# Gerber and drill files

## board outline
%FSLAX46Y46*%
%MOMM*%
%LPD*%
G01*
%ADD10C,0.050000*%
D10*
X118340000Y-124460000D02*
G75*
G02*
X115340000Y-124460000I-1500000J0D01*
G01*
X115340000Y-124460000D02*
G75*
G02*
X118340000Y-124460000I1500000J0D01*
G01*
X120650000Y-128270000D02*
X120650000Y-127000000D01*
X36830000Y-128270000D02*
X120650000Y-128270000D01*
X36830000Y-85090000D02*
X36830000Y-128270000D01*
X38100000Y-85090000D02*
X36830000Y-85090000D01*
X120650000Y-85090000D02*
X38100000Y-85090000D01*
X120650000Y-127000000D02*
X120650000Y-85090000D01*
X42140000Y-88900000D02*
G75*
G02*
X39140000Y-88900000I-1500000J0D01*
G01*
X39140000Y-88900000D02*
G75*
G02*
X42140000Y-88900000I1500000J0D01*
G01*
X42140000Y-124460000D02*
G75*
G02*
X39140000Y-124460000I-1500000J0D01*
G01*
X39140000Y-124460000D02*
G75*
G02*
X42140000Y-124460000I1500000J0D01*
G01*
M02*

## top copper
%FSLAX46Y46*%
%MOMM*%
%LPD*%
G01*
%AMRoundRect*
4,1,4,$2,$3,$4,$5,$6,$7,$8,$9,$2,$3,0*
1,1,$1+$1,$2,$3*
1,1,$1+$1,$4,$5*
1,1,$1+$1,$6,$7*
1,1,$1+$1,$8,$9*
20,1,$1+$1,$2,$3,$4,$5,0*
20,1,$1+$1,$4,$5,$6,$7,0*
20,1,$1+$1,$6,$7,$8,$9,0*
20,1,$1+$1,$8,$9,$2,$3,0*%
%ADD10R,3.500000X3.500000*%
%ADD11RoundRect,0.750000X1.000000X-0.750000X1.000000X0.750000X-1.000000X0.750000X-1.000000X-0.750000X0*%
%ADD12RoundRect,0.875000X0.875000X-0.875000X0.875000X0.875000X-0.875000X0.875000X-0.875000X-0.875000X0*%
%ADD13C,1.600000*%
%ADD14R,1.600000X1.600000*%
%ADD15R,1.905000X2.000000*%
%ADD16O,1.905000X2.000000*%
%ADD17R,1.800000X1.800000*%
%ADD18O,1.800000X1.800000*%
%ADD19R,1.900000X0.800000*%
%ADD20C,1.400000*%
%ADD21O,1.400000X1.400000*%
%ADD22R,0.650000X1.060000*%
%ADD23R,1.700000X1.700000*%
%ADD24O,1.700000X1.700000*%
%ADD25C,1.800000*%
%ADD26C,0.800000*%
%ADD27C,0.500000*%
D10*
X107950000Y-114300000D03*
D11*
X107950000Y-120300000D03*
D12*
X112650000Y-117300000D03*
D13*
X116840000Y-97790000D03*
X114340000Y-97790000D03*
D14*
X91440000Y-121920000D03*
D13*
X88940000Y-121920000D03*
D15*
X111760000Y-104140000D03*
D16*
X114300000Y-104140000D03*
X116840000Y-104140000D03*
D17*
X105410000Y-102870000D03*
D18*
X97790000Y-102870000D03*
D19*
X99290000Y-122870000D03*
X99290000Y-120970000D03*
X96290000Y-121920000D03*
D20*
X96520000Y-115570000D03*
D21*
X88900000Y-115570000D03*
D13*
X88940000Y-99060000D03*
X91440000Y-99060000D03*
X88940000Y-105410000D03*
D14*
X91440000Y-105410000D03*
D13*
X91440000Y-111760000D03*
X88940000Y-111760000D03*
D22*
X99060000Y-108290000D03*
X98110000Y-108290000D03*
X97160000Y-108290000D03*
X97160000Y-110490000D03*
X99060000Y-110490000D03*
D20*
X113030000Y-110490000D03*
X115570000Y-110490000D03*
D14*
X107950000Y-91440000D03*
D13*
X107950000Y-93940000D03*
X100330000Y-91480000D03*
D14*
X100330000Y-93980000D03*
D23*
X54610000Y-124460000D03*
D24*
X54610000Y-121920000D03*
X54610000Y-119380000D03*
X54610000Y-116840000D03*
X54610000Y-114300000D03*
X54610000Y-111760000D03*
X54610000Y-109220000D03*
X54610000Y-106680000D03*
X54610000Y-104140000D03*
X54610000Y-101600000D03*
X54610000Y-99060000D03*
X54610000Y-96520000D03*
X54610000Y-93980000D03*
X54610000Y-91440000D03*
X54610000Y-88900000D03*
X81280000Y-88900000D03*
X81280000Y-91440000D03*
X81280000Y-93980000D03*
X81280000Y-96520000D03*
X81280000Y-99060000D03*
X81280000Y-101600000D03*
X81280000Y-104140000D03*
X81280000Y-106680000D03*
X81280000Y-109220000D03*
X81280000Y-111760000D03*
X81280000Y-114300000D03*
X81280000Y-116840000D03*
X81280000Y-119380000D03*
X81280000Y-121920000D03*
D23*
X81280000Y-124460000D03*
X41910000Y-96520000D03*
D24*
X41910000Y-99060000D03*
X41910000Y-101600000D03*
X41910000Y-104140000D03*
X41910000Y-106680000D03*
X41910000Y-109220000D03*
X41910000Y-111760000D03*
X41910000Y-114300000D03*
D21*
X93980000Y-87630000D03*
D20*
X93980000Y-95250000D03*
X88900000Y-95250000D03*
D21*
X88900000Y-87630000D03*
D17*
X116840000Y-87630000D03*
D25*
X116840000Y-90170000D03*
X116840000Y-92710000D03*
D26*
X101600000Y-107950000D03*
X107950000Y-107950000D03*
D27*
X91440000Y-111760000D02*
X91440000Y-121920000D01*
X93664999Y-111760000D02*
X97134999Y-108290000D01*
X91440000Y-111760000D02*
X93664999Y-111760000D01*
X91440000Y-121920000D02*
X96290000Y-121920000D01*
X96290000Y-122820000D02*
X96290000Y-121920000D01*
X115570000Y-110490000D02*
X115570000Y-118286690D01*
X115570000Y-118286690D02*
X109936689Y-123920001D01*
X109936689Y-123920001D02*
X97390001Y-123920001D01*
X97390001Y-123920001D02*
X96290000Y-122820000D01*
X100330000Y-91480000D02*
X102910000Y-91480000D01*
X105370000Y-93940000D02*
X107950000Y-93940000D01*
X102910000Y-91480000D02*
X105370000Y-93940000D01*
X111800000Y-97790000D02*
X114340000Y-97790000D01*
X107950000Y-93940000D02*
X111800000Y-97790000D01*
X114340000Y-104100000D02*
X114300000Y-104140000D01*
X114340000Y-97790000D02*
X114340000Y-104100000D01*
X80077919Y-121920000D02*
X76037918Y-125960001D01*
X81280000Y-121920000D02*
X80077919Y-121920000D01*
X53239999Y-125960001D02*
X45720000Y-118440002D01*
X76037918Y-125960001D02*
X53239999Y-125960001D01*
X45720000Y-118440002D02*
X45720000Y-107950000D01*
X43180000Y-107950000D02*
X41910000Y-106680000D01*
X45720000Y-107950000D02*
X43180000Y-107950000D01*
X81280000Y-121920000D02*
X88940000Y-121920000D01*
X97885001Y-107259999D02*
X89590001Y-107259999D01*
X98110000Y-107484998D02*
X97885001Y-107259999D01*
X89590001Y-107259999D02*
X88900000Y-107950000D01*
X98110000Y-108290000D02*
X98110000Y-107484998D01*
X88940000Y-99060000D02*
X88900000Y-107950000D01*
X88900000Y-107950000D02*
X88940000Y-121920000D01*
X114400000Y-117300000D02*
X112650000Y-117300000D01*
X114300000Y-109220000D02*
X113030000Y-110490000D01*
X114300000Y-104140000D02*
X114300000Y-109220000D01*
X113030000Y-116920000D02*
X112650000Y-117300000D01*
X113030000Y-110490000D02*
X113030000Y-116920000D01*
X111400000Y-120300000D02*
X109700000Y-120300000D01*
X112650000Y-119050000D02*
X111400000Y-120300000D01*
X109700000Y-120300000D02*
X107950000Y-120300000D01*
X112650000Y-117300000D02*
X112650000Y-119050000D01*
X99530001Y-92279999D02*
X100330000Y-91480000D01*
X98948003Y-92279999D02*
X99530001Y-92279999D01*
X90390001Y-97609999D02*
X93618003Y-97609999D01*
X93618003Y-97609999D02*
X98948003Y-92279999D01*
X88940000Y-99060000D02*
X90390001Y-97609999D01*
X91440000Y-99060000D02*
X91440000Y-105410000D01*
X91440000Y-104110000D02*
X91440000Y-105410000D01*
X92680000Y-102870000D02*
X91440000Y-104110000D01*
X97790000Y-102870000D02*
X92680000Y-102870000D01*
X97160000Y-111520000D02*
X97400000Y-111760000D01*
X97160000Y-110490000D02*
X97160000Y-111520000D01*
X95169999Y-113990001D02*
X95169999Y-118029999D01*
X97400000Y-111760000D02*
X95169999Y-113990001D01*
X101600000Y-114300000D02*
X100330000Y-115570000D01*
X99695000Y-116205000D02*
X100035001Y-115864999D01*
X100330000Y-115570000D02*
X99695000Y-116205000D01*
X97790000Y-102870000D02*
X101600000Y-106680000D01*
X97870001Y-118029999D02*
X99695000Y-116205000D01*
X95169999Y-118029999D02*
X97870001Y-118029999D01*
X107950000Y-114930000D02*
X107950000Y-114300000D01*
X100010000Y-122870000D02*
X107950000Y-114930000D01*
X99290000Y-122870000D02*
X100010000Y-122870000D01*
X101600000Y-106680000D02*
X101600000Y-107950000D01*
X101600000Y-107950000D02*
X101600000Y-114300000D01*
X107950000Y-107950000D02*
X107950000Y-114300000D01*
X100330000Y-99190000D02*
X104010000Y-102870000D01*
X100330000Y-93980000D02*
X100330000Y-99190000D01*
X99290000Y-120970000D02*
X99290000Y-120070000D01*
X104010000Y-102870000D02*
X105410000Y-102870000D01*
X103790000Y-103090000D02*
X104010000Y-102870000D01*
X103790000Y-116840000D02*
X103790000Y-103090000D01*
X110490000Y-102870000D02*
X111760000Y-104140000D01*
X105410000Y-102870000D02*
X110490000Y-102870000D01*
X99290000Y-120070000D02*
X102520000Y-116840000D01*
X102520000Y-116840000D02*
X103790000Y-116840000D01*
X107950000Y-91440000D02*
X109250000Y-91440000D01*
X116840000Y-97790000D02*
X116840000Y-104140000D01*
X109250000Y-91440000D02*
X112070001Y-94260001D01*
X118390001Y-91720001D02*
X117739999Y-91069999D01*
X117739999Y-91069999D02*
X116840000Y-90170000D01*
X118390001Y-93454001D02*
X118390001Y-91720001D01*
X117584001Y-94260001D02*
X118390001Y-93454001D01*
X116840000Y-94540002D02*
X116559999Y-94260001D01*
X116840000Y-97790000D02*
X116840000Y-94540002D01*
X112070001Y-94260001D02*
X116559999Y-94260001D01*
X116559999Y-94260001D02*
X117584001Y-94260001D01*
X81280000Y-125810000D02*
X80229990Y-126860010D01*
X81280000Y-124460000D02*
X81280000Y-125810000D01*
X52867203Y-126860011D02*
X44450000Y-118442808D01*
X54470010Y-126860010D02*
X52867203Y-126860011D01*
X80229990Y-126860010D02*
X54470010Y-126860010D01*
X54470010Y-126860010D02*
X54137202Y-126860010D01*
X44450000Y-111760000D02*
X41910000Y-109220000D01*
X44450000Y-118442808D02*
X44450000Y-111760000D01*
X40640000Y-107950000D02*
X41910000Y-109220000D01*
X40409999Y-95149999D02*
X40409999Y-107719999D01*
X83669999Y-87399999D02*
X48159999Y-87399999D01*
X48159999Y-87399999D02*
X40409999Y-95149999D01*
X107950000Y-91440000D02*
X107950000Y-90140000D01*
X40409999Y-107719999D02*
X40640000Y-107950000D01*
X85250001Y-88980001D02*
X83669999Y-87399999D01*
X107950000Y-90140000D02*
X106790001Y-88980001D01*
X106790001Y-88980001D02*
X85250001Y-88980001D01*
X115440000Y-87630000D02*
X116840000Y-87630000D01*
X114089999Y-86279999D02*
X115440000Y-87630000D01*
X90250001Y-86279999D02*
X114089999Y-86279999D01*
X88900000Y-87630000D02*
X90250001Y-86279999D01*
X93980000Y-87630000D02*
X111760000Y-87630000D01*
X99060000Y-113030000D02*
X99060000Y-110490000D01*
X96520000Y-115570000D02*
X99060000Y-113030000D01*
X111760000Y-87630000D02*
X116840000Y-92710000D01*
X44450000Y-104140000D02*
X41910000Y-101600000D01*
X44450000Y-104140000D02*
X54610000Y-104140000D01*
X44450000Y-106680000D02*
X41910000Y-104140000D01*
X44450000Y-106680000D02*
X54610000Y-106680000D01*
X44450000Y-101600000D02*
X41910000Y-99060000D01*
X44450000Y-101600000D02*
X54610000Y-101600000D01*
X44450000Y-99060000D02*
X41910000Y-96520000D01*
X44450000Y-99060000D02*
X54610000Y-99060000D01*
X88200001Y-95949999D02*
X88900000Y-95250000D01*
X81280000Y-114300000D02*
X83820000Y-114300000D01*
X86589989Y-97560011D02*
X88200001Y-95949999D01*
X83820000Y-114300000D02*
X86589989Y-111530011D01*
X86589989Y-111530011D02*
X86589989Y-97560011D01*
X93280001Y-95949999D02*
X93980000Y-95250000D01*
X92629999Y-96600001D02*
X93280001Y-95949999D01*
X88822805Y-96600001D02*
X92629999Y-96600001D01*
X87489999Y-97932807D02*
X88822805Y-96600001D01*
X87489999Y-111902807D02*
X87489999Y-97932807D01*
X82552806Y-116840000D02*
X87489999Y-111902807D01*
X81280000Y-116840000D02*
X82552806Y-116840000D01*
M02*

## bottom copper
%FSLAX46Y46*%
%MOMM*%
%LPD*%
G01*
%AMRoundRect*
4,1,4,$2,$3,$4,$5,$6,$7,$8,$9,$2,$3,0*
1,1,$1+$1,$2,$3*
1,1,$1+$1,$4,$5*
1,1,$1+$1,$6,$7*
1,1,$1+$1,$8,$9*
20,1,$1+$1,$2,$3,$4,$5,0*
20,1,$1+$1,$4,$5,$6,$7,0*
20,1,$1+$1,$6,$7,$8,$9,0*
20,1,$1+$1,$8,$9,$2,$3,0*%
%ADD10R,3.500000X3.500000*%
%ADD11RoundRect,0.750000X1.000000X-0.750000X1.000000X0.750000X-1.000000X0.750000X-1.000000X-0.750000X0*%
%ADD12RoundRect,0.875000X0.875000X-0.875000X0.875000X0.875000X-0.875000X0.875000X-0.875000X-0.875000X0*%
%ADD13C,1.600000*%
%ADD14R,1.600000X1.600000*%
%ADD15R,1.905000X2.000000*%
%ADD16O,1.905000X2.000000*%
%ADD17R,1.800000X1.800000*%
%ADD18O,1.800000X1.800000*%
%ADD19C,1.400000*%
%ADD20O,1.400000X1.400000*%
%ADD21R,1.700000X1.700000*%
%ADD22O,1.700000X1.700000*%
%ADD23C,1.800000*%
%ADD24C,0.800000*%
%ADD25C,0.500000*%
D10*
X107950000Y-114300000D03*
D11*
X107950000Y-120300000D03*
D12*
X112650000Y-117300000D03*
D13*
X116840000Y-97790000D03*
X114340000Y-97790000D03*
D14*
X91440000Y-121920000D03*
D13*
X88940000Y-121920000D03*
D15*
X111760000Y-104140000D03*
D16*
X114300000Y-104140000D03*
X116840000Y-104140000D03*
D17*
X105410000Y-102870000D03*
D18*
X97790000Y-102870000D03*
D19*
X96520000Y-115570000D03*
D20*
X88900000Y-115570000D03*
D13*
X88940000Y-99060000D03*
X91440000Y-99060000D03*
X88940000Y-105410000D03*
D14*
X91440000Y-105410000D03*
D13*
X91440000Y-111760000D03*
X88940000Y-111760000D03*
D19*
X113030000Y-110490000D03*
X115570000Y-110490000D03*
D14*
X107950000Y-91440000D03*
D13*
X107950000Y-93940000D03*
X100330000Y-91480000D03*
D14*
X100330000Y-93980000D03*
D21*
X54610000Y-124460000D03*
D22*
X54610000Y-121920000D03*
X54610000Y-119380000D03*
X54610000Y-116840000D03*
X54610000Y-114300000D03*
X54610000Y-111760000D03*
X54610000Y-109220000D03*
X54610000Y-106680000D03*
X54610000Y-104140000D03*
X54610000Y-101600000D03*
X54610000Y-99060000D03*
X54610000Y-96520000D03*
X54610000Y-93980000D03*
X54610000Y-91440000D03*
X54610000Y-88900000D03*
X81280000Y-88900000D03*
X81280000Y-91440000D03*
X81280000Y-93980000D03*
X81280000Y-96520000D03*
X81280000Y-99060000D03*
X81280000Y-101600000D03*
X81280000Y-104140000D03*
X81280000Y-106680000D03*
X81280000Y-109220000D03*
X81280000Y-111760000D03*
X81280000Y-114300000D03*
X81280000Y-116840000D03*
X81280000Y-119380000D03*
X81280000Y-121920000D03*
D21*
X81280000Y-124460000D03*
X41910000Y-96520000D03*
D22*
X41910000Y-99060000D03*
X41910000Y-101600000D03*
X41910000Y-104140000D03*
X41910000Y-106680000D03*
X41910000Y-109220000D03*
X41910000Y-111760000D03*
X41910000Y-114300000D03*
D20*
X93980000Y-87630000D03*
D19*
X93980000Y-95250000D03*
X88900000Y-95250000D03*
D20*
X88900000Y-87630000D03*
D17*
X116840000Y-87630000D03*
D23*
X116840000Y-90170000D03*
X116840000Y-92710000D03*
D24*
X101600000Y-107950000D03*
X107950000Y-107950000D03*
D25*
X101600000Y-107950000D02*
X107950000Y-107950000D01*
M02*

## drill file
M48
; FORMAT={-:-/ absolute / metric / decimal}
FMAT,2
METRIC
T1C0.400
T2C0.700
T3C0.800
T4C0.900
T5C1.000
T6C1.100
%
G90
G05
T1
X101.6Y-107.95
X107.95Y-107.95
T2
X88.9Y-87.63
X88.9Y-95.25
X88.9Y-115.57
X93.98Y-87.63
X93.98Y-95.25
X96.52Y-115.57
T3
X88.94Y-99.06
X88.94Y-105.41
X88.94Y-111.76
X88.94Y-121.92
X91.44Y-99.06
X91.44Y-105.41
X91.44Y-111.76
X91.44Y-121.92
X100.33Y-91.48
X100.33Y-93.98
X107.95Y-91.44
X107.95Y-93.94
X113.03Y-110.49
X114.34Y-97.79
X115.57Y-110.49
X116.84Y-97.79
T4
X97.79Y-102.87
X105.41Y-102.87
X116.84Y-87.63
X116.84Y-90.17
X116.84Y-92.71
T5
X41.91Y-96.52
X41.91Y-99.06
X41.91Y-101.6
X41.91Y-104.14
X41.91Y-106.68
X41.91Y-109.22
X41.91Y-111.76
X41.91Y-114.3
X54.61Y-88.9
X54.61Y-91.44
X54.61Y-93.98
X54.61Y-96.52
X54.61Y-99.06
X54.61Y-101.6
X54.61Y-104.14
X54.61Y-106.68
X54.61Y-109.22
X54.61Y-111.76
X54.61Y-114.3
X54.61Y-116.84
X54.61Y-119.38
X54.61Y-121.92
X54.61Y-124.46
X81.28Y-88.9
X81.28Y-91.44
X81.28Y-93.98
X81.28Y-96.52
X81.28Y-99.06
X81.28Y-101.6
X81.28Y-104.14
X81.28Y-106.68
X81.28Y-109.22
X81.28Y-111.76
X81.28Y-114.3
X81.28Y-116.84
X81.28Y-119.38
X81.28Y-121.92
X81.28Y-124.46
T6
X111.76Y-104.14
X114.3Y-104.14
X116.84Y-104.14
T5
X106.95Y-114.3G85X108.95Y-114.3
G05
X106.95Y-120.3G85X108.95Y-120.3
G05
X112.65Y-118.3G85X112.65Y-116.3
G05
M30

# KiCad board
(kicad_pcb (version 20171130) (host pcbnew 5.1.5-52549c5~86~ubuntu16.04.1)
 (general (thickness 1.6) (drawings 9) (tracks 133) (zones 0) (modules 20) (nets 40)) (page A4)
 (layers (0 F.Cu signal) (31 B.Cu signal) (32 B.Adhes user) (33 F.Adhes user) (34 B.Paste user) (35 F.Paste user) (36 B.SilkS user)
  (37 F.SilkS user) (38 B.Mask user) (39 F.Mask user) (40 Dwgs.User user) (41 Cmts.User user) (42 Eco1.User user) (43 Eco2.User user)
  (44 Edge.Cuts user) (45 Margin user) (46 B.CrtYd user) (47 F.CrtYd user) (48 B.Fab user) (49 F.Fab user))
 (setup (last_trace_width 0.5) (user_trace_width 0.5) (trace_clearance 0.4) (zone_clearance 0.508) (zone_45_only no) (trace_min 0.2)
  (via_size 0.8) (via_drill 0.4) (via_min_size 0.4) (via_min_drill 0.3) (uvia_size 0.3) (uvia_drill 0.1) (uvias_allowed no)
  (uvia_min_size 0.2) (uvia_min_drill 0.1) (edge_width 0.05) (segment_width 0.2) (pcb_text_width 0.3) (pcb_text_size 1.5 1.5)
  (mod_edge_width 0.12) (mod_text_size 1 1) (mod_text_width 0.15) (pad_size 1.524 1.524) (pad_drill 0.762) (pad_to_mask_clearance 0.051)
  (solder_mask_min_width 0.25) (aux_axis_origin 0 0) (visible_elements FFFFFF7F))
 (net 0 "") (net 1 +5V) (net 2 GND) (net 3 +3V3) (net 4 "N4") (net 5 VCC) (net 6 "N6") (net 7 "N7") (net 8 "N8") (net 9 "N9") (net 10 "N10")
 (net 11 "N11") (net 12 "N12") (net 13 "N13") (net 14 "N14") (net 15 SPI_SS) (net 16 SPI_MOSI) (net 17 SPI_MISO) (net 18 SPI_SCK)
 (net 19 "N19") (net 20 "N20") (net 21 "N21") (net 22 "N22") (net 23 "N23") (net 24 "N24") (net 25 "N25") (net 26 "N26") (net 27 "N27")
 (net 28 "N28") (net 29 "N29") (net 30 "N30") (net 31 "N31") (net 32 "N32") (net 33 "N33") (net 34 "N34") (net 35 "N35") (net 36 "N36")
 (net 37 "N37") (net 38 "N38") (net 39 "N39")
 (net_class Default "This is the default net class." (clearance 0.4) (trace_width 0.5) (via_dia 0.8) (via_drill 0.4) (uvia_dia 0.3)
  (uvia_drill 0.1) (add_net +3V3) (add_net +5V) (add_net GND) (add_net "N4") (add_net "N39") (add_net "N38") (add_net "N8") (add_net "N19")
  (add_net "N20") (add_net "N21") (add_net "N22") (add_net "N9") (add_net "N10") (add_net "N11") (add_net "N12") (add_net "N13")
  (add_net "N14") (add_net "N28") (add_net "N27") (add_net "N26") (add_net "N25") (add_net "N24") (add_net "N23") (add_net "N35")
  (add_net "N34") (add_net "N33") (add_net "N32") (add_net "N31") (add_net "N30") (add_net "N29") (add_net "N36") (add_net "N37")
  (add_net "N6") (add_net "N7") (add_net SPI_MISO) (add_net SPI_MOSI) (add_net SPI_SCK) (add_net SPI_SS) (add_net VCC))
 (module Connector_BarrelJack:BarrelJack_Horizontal (layer F.Cu) (at 107.95 114.3 90)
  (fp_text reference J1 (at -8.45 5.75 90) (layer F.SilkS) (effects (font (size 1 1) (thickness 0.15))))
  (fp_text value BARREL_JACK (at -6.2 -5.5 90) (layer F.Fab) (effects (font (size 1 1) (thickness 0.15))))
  (pad 1 thru_hole rect (at 0 0 90) (size 3.5 3.5) (drill oval 1 3) (layers *.Cu *.Mask) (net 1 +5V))
  (pad 2 thru_hole roundrect (at -6 0 90) (size 3 3.5) (drill oval 1 3) (layers *.Cu *.Mask) (roundrect_rratio 0.25) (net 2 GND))
  (pad 3 thru_hole roundrect (at -3 4.7 90) (size 3.5 3.5) (drill oval 3 1) (layers *.Cu *.Mask) (roundrect_rratio 0.25) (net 2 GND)))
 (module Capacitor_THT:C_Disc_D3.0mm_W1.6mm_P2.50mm (layer F.Cu) (at 116.84 97.79 180)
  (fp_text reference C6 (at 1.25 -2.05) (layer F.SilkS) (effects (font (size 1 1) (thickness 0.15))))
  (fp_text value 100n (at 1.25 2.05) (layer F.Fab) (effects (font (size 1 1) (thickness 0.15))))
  (pad 1 thru_hole circle (at 0 0 180) (size 1.6 1.6) (drill 0.8) (layers *.Cu *.Mask) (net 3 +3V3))
  (pad 2 thru_hole circle (at 2.5 0 180) (size 1.6 1.6) (drill 0.8) (layers *.Cu *.Mask) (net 2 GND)))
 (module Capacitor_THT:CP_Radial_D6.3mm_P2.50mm (layer F.Cu) (at 91.44 121.92 180)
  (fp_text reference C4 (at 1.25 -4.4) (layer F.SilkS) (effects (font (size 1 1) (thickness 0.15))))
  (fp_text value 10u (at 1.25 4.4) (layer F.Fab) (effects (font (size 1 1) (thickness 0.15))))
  (pad 1 thru_hole rect (at 0 0 180) (size 1.6 1.6) (drill 0.8) (layers *.Cu *.Mask) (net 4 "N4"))
  (pad 2 thru_hole circle (at 2.5 0 180) (size 1.6 1.6) (drill 0.8) (layers *.Cu *.Mask) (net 2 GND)))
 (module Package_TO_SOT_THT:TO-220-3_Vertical (layer F.Cu) (at 111.76 104.14)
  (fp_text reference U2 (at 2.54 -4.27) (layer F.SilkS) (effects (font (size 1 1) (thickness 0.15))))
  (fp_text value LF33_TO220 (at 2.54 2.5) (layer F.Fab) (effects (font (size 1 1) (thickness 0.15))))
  (pad 1 thru_hole rect (at 0 0) (size 1.905 2) (drill 1.1) (layers *.Cu *.Mask) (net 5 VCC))
  (pad 2 thru_hole oval (at 2.54 0) (size 1.905 2) (drill 1.1) (layers *.Cu *.Mask) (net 2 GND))
  (pad 3 thru_hole oval (at 5.08 0) (size 1.905 2) (drill 1.1) (layers *.Cu *.Mask) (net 3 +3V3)))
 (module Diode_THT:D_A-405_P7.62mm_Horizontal (layer F.Cu) (at 105.41 102.87 180)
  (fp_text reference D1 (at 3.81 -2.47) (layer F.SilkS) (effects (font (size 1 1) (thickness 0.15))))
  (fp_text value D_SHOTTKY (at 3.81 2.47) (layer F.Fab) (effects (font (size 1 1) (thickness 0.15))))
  (pad 1 thru_hole rect (at 0 0 180) (size 1.8 1.8) (drill 0.9) (layers *.Cu *.Mask) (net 5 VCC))
  (pad 2 thru_hole oval (at 7.62 0 180) (size 1.8 1.8) (drill 0.9) (layers *.Cu *.Mask) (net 1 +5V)))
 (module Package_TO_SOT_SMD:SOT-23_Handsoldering (layer F.Cu) (at 97.79 121.92 180)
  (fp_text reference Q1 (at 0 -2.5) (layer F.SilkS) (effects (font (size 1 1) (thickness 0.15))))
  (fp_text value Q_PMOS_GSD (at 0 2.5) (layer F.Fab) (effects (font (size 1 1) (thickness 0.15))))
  (pad 1 smd rect (at -1.5 -0.95 180) (size 1.9 0.8) (layers F.Cu F.Paste F.Mask) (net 1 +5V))
  (pad 2 smd rect (at -1.5 0.95 180) (size 1.9 0.8) (layers F.Cu F.Paste F.Mask) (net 5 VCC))
  (pad 3 smd rect (at 1.5 0 180) (size 1.9 0.8) (layers F.Cu F.Paste F.Mask) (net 4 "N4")))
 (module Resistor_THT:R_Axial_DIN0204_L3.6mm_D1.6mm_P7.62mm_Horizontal (layer F.Cu) (at 96.52 115.57 180)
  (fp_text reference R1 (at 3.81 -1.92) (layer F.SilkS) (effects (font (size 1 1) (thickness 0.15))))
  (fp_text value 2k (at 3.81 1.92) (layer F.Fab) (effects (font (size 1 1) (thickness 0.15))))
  (pad 1 thru_hole circle (at 0 0 180) (size 1.4 1.4) (drill 0.7) (layers *.Cu *.Mask) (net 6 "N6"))
  (pad 2 thru_hole oval (at 7.62 0 180) (size 1.4 1.4) (drill 0.7) (layers *.Cu *.Mask) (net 2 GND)))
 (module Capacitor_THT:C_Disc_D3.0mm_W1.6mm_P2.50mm (layer F.Cu) (at 91.44 99.06 180)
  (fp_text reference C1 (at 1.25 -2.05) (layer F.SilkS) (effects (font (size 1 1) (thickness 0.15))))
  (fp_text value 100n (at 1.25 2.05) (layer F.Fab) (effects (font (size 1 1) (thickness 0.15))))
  (pad 2 thru_hole circle (at 2.5 0 180) (size 1.6 1.6) (drill 0.8) (layers *.Cu *.Mask) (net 2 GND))
  (pad 1 thru_hole circle (at 0 0 180) (size 1.6 1.6) (drill 0.8) (layers *.Cu *.Mask) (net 1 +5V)))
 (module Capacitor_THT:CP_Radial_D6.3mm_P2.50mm (layer F.Cu) (at 91.44 105.41 180)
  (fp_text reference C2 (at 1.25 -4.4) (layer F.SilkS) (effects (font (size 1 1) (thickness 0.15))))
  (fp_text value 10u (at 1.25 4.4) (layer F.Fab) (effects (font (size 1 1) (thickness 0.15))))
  (pad 2 thru_hole circle (at 2.5 0 180) (size 1.6 1.6) (drill 0.8) (layers *.Cu *.Mask) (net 2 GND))
  (pad 1 thru_hole rect (at 0 0 180) (size 1.6 1.6) (drill 0.8) (layers *.Cu *.Mask) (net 1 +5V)))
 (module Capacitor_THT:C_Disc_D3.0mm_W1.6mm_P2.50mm (layer F.Cu) (at 91.44 111.76 180)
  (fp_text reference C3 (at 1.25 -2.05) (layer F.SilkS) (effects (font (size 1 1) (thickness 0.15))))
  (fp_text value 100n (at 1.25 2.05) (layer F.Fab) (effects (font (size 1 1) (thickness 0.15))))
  (pad 1 thru_hole circle (at 0 0 180) (size 1.6 1.6) (drill 0.8) (layers *.Cu *.Mask) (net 4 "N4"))
  (pad 2 thru_hole circle (at 2.5 0 180) (size 1.6 1.6) (drill 0.8) (layers *.Cu *.Mask) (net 2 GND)))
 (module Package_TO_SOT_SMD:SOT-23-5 (layer F.Cu) (at 98.11 109.39 270)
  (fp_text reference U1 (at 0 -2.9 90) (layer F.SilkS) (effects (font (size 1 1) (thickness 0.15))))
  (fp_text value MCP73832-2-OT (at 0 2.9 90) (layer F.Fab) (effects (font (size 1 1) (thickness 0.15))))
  (pad 1 smd rect (at -1.1 -0.95 270) (size 1.06 0.65) (layers F.Cu F.Paste F.Mask) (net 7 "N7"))
  (pad 2 smd rect (at -1.1 0 270) (size 1.06 0.65) (layers F.Cu F.Paste F.Mask) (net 2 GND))
  (pad 3 smd rect (at -1.1 0.95 270) (size 1.06 0.65) (layers F.Cu F.Paste F.Mask) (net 4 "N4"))
  (pad 4 smd rect (at 1.1 0.95 270) (size 1.06 0.65) (layers F.Cu F.Paste F.Mask) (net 1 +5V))
  (pad 5 smd rect (at 1.1 -0.95 270) (size 1.06 0.65) (layers F.Cu F.Paste F.Mask) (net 6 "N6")))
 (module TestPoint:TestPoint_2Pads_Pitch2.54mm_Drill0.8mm (layer F.Cu) (at 115.57 110.49 180)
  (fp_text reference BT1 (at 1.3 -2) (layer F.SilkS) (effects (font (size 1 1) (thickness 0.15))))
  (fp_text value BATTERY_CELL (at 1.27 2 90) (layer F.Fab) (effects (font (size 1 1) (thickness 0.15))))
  (pad 2 thru_hole circle (at 2.54 0 180) (size 1.4 1.4) (drill 0.8) (layers *.Cu *.Mask) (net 2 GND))
  (pad 1 thru_hole circle (at 0 0 180) (size 1.4 1.4) (drill 0.8) (layers *.Cu *.Mask) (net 4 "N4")))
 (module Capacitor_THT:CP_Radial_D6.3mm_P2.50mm (layer F.Cu) (at 107.95 91.44 270)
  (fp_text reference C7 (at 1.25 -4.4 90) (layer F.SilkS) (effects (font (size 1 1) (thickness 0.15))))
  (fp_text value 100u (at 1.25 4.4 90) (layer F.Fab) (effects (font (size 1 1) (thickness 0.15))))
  (pad 1 thru_hole rect (at 0 0 270) (size 1.6 1.6) (drill 0.8) (layers *.Cu *.Mask) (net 3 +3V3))
  (pad 2 thru_hole circle (at 2.5 0 270) (size 1.6 1.6) (drill 0.8) (layers *.Cu *.Mask) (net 2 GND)))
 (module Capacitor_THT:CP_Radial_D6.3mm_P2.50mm (layer F.Cu) (at 100.33 93.98 90)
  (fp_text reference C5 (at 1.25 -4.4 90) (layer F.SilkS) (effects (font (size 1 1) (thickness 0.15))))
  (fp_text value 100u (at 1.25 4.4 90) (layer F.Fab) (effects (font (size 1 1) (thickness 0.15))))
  (pad 2 thru_hole circle (at 2.5 0 90) (size 1.6 1.6) (drill 0.8) (layers *.Cu *.Mask) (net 2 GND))
  (pad 1 thru_hole rect (at 0 0 90) (size 1.6 1.6) (drill 0.8) (layers *.Cu *.Mask) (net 5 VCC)))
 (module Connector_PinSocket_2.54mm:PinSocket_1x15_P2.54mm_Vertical (layer F.Cu) (at 54.61 124.46 180)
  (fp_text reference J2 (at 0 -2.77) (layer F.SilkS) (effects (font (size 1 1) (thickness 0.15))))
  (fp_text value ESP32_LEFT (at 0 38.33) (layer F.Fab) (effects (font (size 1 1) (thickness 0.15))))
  (pad 1 thru_hole rect (at 0 0 180) (size 1.7 1.7) (drill 1) (layers *.Cu *.Mask) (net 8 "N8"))
  (pad 2 thru_hole oval (at 0 2.54 180) (size 1.7 1.7) (drill 1) (layers *.Cu *.Mask) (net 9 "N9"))
  (pad 3 thru_hole oval (at 0 5.08 180) (size 1.7 1.7) (drill 1) (layers *.Cu *.Mask) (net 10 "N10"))
  (pad 4 thru_hole oval (at 0 7.62 180) (size 1.7 1.7) (drill 1) (layers *.Cu *.Mask) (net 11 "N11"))
  (pad 5 thru_hole oval (at 0 10.16 180) (size 1.7 1.7) (drill 1) (layers *.Cu *.Mask) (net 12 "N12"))
  (pad 6 thru_hole oval (at 0 12.7 180) (size 1.7 1.7) (drill 1) (layers *.Cu *.Mask) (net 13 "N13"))
  (pad 7 thru_hole oval (at 0 15.24 180) (size 1.7 1.7) (drill 1) (layers *.Cu *.Mask) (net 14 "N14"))
  (pad 8 thru_hole oval (at 0 17.78 180) (size 1.7 1.7) (drill 1) (layers *.Cu *.Mask) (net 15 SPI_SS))
  (pad 9 thru_hole oval (at 0 20.32 180) (size 1.7 1.7) (drill 1) (layers *.Cu *.Mask) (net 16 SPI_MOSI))
  (pad 10 thru_hole oval (at 0 22.86 180) (size 1.7 1.7) (drill 1) (layers *.Cu *.Mask) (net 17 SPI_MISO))
  (pad 11 thru_hole oval (at 0 25.4 180) (size 1.7 1.7) (drill 1) (layers *.Cu *.Mask) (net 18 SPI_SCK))
  (pad 12 thru_hole oval (at 0 27.94 180) (size 1.7 1.7) (drill 1) (layers *.Cu *.Mask) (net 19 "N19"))
  (pad 13 thru_hole oval (at 0 30.48 180) (size 1.7 1.7) (drill 1) (layers *.Cu *.Mask) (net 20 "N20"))
  (pad 14 thru_hole oval (at 0 33.02 180) (size 1.7 1.7) (drill 1) (layers *.Cu *.Mask) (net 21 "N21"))
  (pad 15 thru_hole oval (at 0 35.56 180) (size 1.7 1.7) (drill 1) (layers *.Cu *.Mask) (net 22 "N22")))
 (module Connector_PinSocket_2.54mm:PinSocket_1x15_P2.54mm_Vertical (layer F.Cu) (at 81.28 124.46 180)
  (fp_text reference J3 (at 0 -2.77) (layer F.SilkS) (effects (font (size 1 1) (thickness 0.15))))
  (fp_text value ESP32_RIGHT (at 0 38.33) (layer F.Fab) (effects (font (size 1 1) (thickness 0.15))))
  (pad 15 thru_hole oval (at 0 35.56 180) (size 1.7 1.7) (drill 1) (layers *.Cu *.Mask) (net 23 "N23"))
  (pad 14 thru_hole oval (at 0 33.02 180) (size 1.7 1.7) (drill 1) (layers *.Cu *.Mask) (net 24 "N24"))
  (pad 13 thru_hole oval (at 0 30.48 180) (size 1.7 1.7) (drill 1) (layers *.Cu *.Mask) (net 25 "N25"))
  (pad 12 thru_hole oval (at 0 27.94 180) (size 1.7 1.7) (drill 1) (layers *.Cu *.Mask) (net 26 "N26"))
  (pad 11 thru_hole oval (at 0 25.4 180) (size 1.7 1.7) (drill 1) (layers *.Cu *.Mask) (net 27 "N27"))
  (pad 10 thru_hole oval (at 0 22.86 180) (size 1.7 1.7) (drill 1) (layers *.Cu *.Mask) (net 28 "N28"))
  (pad 9 thru_hole oval (at 0 20.32 180) (size 1.7 1.7) (drill 1) (layers *.Cu *.Mask) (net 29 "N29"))
  (pad 8 thru_hole oval (at 0 17.78 180) (size 1.7 1.7) (drill 1) (layers *.Cu *.Mask) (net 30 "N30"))
  (pad 7 thru_hole oval (at 0 15.24 180) (size 1.7 1.7) (drill 1) (layers *.Cu *.Mask) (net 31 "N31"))
  (pad 6 thru_hole oval (at 0 12.7 180) (size 1.7 1.7) (drill 1) (layers *.Cu *.Mask) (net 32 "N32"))
  (pad 5 thru_hole oval (at 0 10.16 180) (size 1.7 1.7) (drill 1) (layers *.Cu *.Mask) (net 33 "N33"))
  (pad 4 thru_hole oval (at 0 7.62 180) (size 1.7 1.7) (drill 1) (layers *.Cu *.Mask) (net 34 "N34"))
  (pad 3 thru_hole oval (at 0 5.08 180) (size 1.7 1.7) (drill 1) (layers *.Cu *.Mask) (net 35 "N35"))
  (pad 2 thru_hole oval (at 0 2.54 180) (size 1.7 1.7) (drill 1) (layers *.Cu *.Mask) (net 2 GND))
  (pad 1 thru_hole rect (at 0 0 180) (size 1.7 1.7) (drill 1) (layers *.Cu *.Mask) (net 3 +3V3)))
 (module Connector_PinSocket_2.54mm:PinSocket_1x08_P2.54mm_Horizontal (layer F.Cu) (at 41.91 96.52)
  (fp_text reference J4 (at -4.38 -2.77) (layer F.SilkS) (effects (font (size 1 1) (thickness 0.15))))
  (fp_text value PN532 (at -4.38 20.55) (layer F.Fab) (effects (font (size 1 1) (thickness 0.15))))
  (pad 1 thru_hole rect (at 0 0) (size 1.7 1.7) (drill 1) (layers *.Cu *.Mask) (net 18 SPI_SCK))
  (pad 2 thru_hole oval (at 0 2.54) (size 1.7 1.7) (drill 1) (layers *.Cu *.Mask) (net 17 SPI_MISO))
  (pad 3 thru_hole oval (at 0 5.08) (size 1.7 1.7) (drill 1) (layers *.Cu *.Mask) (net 16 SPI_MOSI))
  (pad 4 thru_hole oval (at 0 7.62) (size 1.7 1.7) (drill 1) (layers *.Cu *.Mask) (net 15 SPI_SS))
  (pad 5 thru_hole oval (at 0 10.16) (size 1.7 1.7) (drill 1) (layers *.Cu *.Mask) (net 2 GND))
  (pad 6 thru_hole oval (at 0 12.7) (size 1.7 1.7) (drill 1) (layers *.Cu *.Mask) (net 3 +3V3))
  (pad 7 thru_hole oval (at 0 15.24) (size 1.7 1.7) (drill 1) (layers *.Cu *.Mask) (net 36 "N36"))
  (pad 8 thru_hole oval (at 0 17.78) (size 1.7 1.7) (drill 1) (layers *.Cu *.Mask) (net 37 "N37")))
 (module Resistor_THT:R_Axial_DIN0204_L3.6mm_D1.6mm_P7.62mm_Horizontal (layer F.Cu) (at 93.98 95.25 90)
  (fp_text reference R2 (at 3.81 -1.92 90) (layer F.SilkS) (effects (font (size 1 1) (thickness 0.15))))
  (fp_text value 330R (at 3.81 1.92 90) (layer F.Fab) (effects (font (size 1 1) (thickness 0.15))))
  (pad 2 thru_hole oval (at 7.62 0 90) (size 1.4 1.4) (drill 0.7) (layers *.Cu *.Mask) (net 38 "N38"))
  (pad 1 thru_hole circle (at 0 0 90) (size 1.4 1.4) (drill 0.7) (layers *.Cu *.Mask) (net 34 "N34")))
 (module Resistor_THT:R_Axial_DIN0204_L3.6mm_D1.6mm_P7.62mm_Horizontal (layer F.Cu) (at 88.9 95.25 90)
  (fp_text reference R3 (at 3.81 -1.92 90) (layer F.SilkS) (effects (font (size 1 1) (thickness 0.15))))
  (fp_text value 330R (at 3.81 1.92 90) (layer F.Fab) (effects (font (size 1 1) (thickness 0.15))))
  (pad 1 thru_hole circle (at 0 0 90) (size 1.4 1.4) (drill 0.7) (layers *.Cu *.Mask) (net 33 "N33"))
  (pad 2 thru_hole oval (at 7.62 0 90) (size 1.4 1.4) (drill 0.7) (layers *.Cu *.Mask) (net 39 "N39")))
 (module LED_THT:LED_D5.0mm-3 (layer F.Cu) (at 116.84 87.63 270)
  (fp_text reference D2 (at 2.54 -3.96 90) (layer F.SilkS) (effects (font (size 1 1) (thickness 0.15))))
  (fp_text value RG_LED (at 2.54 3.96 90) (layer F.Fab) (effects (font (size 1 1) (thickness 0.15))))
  (pad 1 thru_hole rect (at 0 0 270) (size 1.8 1.8) (drill 0.9) (layers *.Cu *.Mask) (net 39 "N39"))
  (pad 2 thru_hole circle (at 2.54 0 270) (size 1.8 1.8) (drill 0.9) (layers *.Cu *.Mask) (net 3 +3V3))
  (pad 3 thru_hole circle (at 5.08 0 270) (size 1.8 1.8) (drill 0.9) (layers *.Cu *.Mask) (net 38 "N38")))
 (gr_circle (center 116.84 124.46) (end 118.34 124.46) (layer Edge.Cuts) (width 0.05))
 (gr_line (start 120.65 128.27) (end 120.65 127) (layer Edge.Cuts) (width 0.05))
 (gr_line (start 36.83 128.27) (end 120.65 128.27) (layer Edge.Cuts) (width 0.05))
 (gr_line (start 36.83 85.09) (end 36.83 128.27) (layer Edge.Cuts) (width 0.05))
 (gr_line (start 38.1 85.09) (end 36.83 85.09) (layer Edge.Cuts) (width 0.05))
 (gr_line (start 120.65 85.09) (end 38.1 85.09) (layer Edge.Cuts) (width 0.05))
 (gr_line (start 120.65 127) (end 120.65 85.09) (layer Edge.Cuts) (width 0.05))
 (gr_circle (center 40.64 88.9) (end 42.14 88.9) (layer Edge.Cuts) (width 0.05))
 (gr_circle (center 40.64 124.46) (end 42.14 124.46) (layer Edge.Cuts) (width 0.05))
 (segment (start 91.44 111.76) (end 91.44 121.92) (width 0.5) (layer F.Cu) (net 4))
 (segment (start 93.664999 111.76) (end 97.134999 108.29) (width 0.5) (layer F.Cu) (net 4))
 (segment (start 91.44 111.76) (end 93.664999 111.76) (width 0.5) (layer F.Cu) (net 4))
 (segment (start 91.44 121.92) (end 96.29 121.92) (width 0.5) (layer F.Cu) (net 4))
 (segment (start 96.29 122.82) (end 96.29 121.92) (width 0.5) (layer F.Cu) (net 4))
 (segment (start 115.57 110.49) (end 115.57 118.28669) (width 0.5) (layer F.Cu) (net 4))
 (segment (start 115.57 118.28669) (end 109.936689 123.920001) (width 0.5) (layer F.Cu) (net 4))
 (segment (start 109.936689 123.920001) (end 97.390001 123.920001) (width 0.5) (layer F.Cu) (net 4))
 (segment (start 97.390001 123.920001) (end 96.29 122.82) (width 0.5) (layer F.Cu) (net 4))
 (segment (start 100.33 91.48) (end 102.91 91.48) (width 0.5) (layer F.Cu) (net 2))
 (segment (start 105.37 93.94) (end 107.95 93.94) (width 0.5) (layer F.Cu) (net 2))
 (segment (start 102.91 91.48) (end 105.37 93.94) (width 0.5) (layer F.Cu) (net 2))
 (segment (start 111.8 97.79) (end 114.34 97.79) (width 0.5) (layer F.Cu) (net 2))
 (segment (start 107.95 93.94) (end 111.8 97.79) (width 0.5) (layer F.Cu) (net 2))
 (segment (start 114.34 104.1) (end 114.3 104.14) (width 0.5) (layer F.Cu) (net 2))
 (segment (start 114.34 97.79) (end 114.34 104.1) (width 0.5) (layer F.Cu) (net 2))
 (segment (start 80.077919 121.92) (end 76.037918 125.960001) (width 0.5) (layer F.Cu) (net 2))
 (segment (start 81.28 121.92) (end 80.077919 121.92) (width 0.5) (layer F.Cu) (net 2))
 (segment (start 53.239999 125.960001) (end 45.72 118.440002) (width 0.5) (layer F.Cu) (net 2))
 (segment (start 76.037918 125.960001) (end 53.239999 125.960001) (width 0.5) (layer F.Cu) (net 2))
 (segment (start 45.72 118.440002) (end 45.72 107.95) (width 0.5) (layer F.Cu) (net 2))
 (segment (start 43.18 107.95) (end 41.91 106.68) (width 0.5) (layer F.Cu) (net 2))
 (segment (start 45.72 107.95) (end 43.18 107.95) (width 0.5) (layer F.Cu) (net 2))
 (segment (start 81.28 121.92) (end 88.94 121.92) (width 0.5) (layer F.Cu) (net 2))
 (segment (start 97.885001 107.259999) (end 89.590001 107.259999) (width 0.5) (layer F.Cu) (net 2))
 (segment (start 98.11 107.484998) (end 97.885001 107.259999) (width 0.5) (layer F.Cu) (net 2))
 (segment (start 89.590001 107.259999) (end 88.9 107.95) (width 0.5) (layer F.Cu) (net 2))
 (segment (start 98.11 108.29) (end 98.11 107.484998) (width 0.5) (layer F.Cu) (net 2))
 (segment (start 88.94 99.06) (end 88.9 107.95) (width 0.5) (layer F.Cu) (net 2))
 (segment (start 88.9 107.95) (end 88.94 121.92) (width 0.5) (layer F.Cu) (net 2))
 (segment (start 114.4 117.3) (end 112.65 117.3) (width 0.5) (layer F.Cu) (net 2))
 (segment (start 114.3 109.22) (end 113.03 110.49) (width 0.5) (layer F.Cu) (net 2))
 (segment (start 114.3 104.14) (end 114.3 109.22) (width 0.5) (layer F.Cu) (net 2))
 (segment (start 113.03 116.92) (end 112.65 117.3) (width 0.5) (layer F.Cu) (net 2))
 (segment (start 113.03 110.49) (end 113.03 116.92) (width 0.5) (layer F.Cu) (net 2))
 (segment (start 111.4 120.3) (end 109.7 120.3) (width 0.5) (layer F.Cu) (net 2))
 (segment (start 112.65 119.05) (end 111.4 120.3) (width 0.5) (layer F.Cu) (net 2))
 (segment (start 109.7 120.3) (end 107.95 120.3) (width 0.5) (layer F.Cu) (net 2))
 (segment (start 112.65 117.3) (end 112.65 119.05) (width 0.5) (layer F.Cu) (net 2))
 (segment (start 99.530001 92.279999) (end 100.33 91.48) (width 0.5) (layer F.Cu) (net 2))
 (segment (start 98.948003 92.279999) (end 99.530001 92.279999) (width 0.5) (layer F.Cu) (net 2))
 (segment (start 90.390001 97.609999) (end 93.618003 97.609999) (width 0.5) (layer F.Cu) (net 2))
 (segment (start 93.618003 97.609999) (end 98.948003 92.279999) (width 0.5) (layer F.Cu) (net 2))
 (segment (start 88.94 99.06) (end 90.390001 97.609999) (width 0.5) (layer F.Cu) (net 2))
 (segment (start 91.44 99.06) (end 91.44 105.41) (width 0.5) (layer F.Cu) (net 1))
 (segment (start 91.44 104.11) (end 91.44 105.41) (width 0.5) (layer F.Cu) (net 1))
 (segment (start 92.68 102.87) (end 91.44 104.11) (width 0.5) (layer F.Cu) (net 1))
 (segment (start 97.79 102.87) (end 92.68 102.87) (width 0.5) (layer F.Cu) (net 1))
 (segment (start 97.16 111.52) (end 97.4 111.76) (width 0.5) (layer F.Cu) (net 1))
 (segment (start 97.16 110.49) (end 97.16 111.52) (width 0.5) (layer F.Cu) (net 1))
 (segment (start 95.169999 113.990001) (end 95.169999 118.029999) (width 0.5) (layer F.Cu) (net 1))
 (segment (start 97.4 111.76) (end 95.169999 113.990001) (width 0.5) (layer F.Cu) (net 1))
 (segment (start 101.6 114.3) (end 100.33 115.57) (width 0.5) (layer F.Cu) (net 1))
 (segment (start 99.695 116.205) (end 100.035001 115.864999) (width 0.5) (layer F.Cu) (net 1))
 (segment (start 100.33 115.57) (end 99.695 116.205) (width 0.5) (layer F.Cu) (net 1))
 (segment (start 97.79 102.87) (end 101.6 106.68) (width 0.5) (layer F.Cu) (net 1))
 (segment (start 97.870001 118.029999) (end 99.695 116.205) (width 0.5) (layer F.Cu) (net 1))
 (segment (start 95.169999 118.029999) (end 97.870001 118.029999) (width 0.5) (layer F.Cu) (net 1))
 (segment (start 107.95 114.93) (end 107.95 114.3) (width 0.5) (layer F.Cu) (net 1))
 (segment (start 100.01 122.87) (end 107.95 114.93) (width 0.5) (layer F.Cu) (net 1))
 (segment (start 99.29 122.87) (end 100.01 122.87) (width 0.5) (layer F.Cu) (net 1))
 (via (at 101.6 107.95) (size 0.8) (drill 0.4) (layers F.Cu B.Cu) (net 1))
 (segment (start 101.6 106.68) (end 101.6 107.95) (width 0.5) (layer F.Cu) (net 1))
 (segment (start 101.6 107.95) (end 101.6 114.3) (width 0.5) (layer F.Cu) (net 1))
 (via (at 107.95 107.95) (size 0.8) (drill 0.4) (layers F.Cu B.Cu) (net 1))
 (segment (start 101.6 107.95) (end 107.95 107.95) (width 0.5) (layer B.Cu) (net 1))
 (segment (start 107.95 107.95) (end 107.95 114.3) (width 0.5) (layer F.Cu) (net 1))
 (segment (start 100.33 99.19) (end 104.01 102.87) (width 0.5) (layer F.Cu) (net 5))
 (segment (start 100.33 93.98) (end 100.33 99.19) (width 0.5) (layer F.Cu) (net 5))
 (segment (start 99.29 120.97) (end 99.29 120.07) (width 0.5) (layer F.Cu) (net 5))
 (segment (start 104.01 102.87) (end 105.41 102.87) (width 0.5) (layer F.Cu) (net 5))
 (segment (start 103.79 103.09) (end 104.01 102.87) (width 0.5) (layer F.Cu) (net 5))
 (segment (start 103.79 116.84) (end 103.79 103.09) (width 0.5) (layer F.Cu) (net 5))
 (segment (start 110.49 102.87) (end 111.76 104.14) (width 0.5) (layer F.Cu) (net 5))
 (segment (start 105.41 102.87) (end 110.49 102.87) (width 0.5) (layer F.Cu) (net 5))
 (segment (start 99.29 120.07) (end 102.52 116.84) (width 0.5) (layer F.Cu) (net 5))
 (segment (start 102.52 116.84) (end 103.79 116.84) (width 0.5) (layer F.Cu) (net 5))
 (segment (start 107.95 91.44) (end 109.25 91.44) (width 0.5) (layer F.Cu) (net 3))
 (segment (start 116.84 97.79) (end 116.84 104.14) (width 0.5) (layer F.Cu) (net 3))
 (segment (start 109.25 91.44) (end 112.070001 94.260001) (width 0.5) (layer F.Cu) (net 3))
 (segment (start 118.390001 91.720001) (end 117.739999 91.069999) (width 0.5) (layer F.Cu) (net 3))
 (segment (start 117.739999 91.069999) (end 116.84 90.17) (width 0.5) (layer F.Cu) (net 3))
 (segment (start 118.390001 93.454001) (end 118.390001 91.720001) (width 0.5) (layer F.Cu) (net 3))
 (segment (start 117.584001 94.260001) (end 118.390001 93.454001) (width 0.5) (layer F.Cu) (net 3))
 (segment (start 116.84 94.540002) (end 116.559999 94.260001) (width 0.5) (layer F.Cu) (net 3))
 (segment (start 116.84 97.79) (end 116.84 94.540002) (width 0.5) (layer F.Cu) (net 3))
 (segment (start 112.070001 94.260001) (end 116.559999 94.260001) (width 0.5) (layer F.Cu) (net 3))
 (segment (start 116.559999 94.260001) (end 117.584001 94.260001) (width 0.5) (layer F.Cu) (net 3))
 (segment (start 81.28 125.81) (end 80.22999 126.86001) (width 0.5) (layer F.Cu) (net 3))
 (segment (start 81.28 124.46) (end 81.28 125.81) (width 0.5) (layer F.Cu) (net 3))
 (segment (start 52.867203 126.860011) (end 44.45 118.442808) (width 0.5) (layer F.Cu) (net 3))
 (segment (start 54.47001 126.86001) (end 52.867203 126.860011) (width 0.5) (layer F.Cu) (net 3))
 (segment (start 80.22999 126.86001) (end 54.47001 126.86001) (width 0.5) (layer F.Cu) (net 3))
 (segment (start 54.47001 126.86001) (end 54.137202 126.86001) (width 0.5) (layer F.Cu) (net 3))
 (segment (start 44.45 111.76) (end 41.91 109.22) (width 0.5) (layer F.Cu) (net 3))
 (segment (start 44.45 118.442808) (end 44.45 111.76) (width 0.5) (layer F.Cu) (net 3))
 (segment (start 40.64 107.95) (end 41.91 109.22) (width 0.5) (layer F.Cu) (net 3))
 (segment (start 40.409999 95.149999) (end 40.409999 107.719999) (width 0.5) (layer F.Cu) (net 3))
 (segment (start 83.669999 87.399999) (end 48.159999 87.399999) (width 0.5) (layer F.Cu) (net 3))
 (segment (start 48.159999 87.399999) (end 40.409999 95.149999) (width 0.5) (layer F.Cu) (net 3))
 (segment (start 107.95 91.44) (end 107.95 90.14) (width 0.5) (layer F.Cu) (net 3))
 (segment (start 40.409999 107.719999) (end 40.64 107.95) (width 0.5) (layer F.Cu) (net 3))
 (segment (start 85.250001 88.980001) (end 83.669999 87.399999) (width 0.5) (layer F.Cu) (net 3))
 (segment (start 107.95 90.14) (end 106.790001 88.980001) (width 0.5) (layer F.Cu) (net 3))
 (segment (start 106.790001 88.980001) (end 85.250001 88.980001) (width 0.5) (layer F.Cu) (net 3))
 (segment (start 115.44 87.63) (end 116.84 87.63) (width 0.5) (layer F.Cu) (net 39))
 (segment (start 114.089999 86.279999) (end 115.44 87.63) (width 0.5) (layer F.Cu) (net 39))
 (segment (start 90.250001 86.279999) (end 114.089999 86.279999) (width 0.5) (layer F.Cu) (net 39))
 (segment (start 88.9 87.63) (end 90.250001 86.279999) (width 0.5) (layer F.Cu) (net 39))
 (segment (start 93.98 87.63) (end 111.76 87.63) (width 0.5) (layer F.Cu) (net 38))
 (segment (start 99.06 113.03) (end 99.06 110.49) (width 0.5) (layer F.Cu) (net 6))
 (segment (start 96.52 115.57) (end 99.06 113.03) (width 0.5) (layer F.Cu) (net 6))
 (segment (start 111.76 87.63) (end 116.84 92.71) (width 0.5) (layer F.Cu) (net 38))
 (segment (start 44.45 104.14) (end 41.91 101.6) (width 0.5) (layer F.Cu) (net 16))
 (segment (start 44.45 104.14) (end 54.61 104.14) (width 0.5) (layer F.Cu) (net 16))
 (segment (start 44.45 106.68) (end 41.91 104.14) (width 0.5) (layer F.Cu) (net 15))
 (segment (start 44.45 106.68) (end 54.61 106.68) (width 0.5) (layer F.Cu) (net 15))
 (segment (start 44.45 101.6) (end 41.91 99.06) (width 0.5) (layer F.Cu) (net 17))
 (segment (start 44.45 101.6) (end 54.61 101.6) (width 0.5) (layer F.Cu) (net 17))
 (segment (start 44.45 99.06) (end 41.91 96.52) (width 0.5) (layer F.Cu) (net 18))
 (segment (start 44.45 99.06) (end 54.61 99.06) (width 0.5) (layer F.Cu) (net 18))
 (segment (start 88.200001 95.949999) (end 88.9 95.25) (width 0.5) (layer F.Cu) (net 33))
 (segment (start 81.28 114.3) (end 83.82 114.3) (width 0.5) (layer F.Cu) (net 33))
 (segment (start 86.589989 97.560011) (end 88.200001 95.949999) (width 0.5) (layer F.Cu) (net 33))
 (segment (start 83.82 114.3) (end 86.589989 111.530011) (width 0.5) (layer F.Cu) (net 33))
 (segment (start 86.589989 111.530011) (end 86.589989 97.560011) (width 0.5) (layer F.Cu) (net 33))
 (segment (start 93.280001 95.949999) (end 93.98 95.25) (width 0.5) (layer F.Cu) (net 34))
 (segment (start 92.629999 96.600001) (end 93.280001 95.949999) (width 0.5) (layer F.Cu) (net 34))
 (segment (start 88.822805 96.600001) (end 92.629999 96.600001) (width 0.5) (layer F.Cu) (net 34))
 (segment (start 87.489999 97.932807) (end 88.822805 96.600001) (width 0.5) (layer F.Cu) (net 34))
 (segment (start 87.489999 111.902807) (end 87.489999 97.932807) (width 0.5) (layer F.Cu) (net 34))
 (segment (start 82.552806 116.84) (end 87.489999 111.902807) (width 0.5) (layer F.Cu) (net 34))
 (segment (start 81.28 116.84) (end 82.552806 116.84) (width 0.5) (layer F.Cu) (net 34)))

